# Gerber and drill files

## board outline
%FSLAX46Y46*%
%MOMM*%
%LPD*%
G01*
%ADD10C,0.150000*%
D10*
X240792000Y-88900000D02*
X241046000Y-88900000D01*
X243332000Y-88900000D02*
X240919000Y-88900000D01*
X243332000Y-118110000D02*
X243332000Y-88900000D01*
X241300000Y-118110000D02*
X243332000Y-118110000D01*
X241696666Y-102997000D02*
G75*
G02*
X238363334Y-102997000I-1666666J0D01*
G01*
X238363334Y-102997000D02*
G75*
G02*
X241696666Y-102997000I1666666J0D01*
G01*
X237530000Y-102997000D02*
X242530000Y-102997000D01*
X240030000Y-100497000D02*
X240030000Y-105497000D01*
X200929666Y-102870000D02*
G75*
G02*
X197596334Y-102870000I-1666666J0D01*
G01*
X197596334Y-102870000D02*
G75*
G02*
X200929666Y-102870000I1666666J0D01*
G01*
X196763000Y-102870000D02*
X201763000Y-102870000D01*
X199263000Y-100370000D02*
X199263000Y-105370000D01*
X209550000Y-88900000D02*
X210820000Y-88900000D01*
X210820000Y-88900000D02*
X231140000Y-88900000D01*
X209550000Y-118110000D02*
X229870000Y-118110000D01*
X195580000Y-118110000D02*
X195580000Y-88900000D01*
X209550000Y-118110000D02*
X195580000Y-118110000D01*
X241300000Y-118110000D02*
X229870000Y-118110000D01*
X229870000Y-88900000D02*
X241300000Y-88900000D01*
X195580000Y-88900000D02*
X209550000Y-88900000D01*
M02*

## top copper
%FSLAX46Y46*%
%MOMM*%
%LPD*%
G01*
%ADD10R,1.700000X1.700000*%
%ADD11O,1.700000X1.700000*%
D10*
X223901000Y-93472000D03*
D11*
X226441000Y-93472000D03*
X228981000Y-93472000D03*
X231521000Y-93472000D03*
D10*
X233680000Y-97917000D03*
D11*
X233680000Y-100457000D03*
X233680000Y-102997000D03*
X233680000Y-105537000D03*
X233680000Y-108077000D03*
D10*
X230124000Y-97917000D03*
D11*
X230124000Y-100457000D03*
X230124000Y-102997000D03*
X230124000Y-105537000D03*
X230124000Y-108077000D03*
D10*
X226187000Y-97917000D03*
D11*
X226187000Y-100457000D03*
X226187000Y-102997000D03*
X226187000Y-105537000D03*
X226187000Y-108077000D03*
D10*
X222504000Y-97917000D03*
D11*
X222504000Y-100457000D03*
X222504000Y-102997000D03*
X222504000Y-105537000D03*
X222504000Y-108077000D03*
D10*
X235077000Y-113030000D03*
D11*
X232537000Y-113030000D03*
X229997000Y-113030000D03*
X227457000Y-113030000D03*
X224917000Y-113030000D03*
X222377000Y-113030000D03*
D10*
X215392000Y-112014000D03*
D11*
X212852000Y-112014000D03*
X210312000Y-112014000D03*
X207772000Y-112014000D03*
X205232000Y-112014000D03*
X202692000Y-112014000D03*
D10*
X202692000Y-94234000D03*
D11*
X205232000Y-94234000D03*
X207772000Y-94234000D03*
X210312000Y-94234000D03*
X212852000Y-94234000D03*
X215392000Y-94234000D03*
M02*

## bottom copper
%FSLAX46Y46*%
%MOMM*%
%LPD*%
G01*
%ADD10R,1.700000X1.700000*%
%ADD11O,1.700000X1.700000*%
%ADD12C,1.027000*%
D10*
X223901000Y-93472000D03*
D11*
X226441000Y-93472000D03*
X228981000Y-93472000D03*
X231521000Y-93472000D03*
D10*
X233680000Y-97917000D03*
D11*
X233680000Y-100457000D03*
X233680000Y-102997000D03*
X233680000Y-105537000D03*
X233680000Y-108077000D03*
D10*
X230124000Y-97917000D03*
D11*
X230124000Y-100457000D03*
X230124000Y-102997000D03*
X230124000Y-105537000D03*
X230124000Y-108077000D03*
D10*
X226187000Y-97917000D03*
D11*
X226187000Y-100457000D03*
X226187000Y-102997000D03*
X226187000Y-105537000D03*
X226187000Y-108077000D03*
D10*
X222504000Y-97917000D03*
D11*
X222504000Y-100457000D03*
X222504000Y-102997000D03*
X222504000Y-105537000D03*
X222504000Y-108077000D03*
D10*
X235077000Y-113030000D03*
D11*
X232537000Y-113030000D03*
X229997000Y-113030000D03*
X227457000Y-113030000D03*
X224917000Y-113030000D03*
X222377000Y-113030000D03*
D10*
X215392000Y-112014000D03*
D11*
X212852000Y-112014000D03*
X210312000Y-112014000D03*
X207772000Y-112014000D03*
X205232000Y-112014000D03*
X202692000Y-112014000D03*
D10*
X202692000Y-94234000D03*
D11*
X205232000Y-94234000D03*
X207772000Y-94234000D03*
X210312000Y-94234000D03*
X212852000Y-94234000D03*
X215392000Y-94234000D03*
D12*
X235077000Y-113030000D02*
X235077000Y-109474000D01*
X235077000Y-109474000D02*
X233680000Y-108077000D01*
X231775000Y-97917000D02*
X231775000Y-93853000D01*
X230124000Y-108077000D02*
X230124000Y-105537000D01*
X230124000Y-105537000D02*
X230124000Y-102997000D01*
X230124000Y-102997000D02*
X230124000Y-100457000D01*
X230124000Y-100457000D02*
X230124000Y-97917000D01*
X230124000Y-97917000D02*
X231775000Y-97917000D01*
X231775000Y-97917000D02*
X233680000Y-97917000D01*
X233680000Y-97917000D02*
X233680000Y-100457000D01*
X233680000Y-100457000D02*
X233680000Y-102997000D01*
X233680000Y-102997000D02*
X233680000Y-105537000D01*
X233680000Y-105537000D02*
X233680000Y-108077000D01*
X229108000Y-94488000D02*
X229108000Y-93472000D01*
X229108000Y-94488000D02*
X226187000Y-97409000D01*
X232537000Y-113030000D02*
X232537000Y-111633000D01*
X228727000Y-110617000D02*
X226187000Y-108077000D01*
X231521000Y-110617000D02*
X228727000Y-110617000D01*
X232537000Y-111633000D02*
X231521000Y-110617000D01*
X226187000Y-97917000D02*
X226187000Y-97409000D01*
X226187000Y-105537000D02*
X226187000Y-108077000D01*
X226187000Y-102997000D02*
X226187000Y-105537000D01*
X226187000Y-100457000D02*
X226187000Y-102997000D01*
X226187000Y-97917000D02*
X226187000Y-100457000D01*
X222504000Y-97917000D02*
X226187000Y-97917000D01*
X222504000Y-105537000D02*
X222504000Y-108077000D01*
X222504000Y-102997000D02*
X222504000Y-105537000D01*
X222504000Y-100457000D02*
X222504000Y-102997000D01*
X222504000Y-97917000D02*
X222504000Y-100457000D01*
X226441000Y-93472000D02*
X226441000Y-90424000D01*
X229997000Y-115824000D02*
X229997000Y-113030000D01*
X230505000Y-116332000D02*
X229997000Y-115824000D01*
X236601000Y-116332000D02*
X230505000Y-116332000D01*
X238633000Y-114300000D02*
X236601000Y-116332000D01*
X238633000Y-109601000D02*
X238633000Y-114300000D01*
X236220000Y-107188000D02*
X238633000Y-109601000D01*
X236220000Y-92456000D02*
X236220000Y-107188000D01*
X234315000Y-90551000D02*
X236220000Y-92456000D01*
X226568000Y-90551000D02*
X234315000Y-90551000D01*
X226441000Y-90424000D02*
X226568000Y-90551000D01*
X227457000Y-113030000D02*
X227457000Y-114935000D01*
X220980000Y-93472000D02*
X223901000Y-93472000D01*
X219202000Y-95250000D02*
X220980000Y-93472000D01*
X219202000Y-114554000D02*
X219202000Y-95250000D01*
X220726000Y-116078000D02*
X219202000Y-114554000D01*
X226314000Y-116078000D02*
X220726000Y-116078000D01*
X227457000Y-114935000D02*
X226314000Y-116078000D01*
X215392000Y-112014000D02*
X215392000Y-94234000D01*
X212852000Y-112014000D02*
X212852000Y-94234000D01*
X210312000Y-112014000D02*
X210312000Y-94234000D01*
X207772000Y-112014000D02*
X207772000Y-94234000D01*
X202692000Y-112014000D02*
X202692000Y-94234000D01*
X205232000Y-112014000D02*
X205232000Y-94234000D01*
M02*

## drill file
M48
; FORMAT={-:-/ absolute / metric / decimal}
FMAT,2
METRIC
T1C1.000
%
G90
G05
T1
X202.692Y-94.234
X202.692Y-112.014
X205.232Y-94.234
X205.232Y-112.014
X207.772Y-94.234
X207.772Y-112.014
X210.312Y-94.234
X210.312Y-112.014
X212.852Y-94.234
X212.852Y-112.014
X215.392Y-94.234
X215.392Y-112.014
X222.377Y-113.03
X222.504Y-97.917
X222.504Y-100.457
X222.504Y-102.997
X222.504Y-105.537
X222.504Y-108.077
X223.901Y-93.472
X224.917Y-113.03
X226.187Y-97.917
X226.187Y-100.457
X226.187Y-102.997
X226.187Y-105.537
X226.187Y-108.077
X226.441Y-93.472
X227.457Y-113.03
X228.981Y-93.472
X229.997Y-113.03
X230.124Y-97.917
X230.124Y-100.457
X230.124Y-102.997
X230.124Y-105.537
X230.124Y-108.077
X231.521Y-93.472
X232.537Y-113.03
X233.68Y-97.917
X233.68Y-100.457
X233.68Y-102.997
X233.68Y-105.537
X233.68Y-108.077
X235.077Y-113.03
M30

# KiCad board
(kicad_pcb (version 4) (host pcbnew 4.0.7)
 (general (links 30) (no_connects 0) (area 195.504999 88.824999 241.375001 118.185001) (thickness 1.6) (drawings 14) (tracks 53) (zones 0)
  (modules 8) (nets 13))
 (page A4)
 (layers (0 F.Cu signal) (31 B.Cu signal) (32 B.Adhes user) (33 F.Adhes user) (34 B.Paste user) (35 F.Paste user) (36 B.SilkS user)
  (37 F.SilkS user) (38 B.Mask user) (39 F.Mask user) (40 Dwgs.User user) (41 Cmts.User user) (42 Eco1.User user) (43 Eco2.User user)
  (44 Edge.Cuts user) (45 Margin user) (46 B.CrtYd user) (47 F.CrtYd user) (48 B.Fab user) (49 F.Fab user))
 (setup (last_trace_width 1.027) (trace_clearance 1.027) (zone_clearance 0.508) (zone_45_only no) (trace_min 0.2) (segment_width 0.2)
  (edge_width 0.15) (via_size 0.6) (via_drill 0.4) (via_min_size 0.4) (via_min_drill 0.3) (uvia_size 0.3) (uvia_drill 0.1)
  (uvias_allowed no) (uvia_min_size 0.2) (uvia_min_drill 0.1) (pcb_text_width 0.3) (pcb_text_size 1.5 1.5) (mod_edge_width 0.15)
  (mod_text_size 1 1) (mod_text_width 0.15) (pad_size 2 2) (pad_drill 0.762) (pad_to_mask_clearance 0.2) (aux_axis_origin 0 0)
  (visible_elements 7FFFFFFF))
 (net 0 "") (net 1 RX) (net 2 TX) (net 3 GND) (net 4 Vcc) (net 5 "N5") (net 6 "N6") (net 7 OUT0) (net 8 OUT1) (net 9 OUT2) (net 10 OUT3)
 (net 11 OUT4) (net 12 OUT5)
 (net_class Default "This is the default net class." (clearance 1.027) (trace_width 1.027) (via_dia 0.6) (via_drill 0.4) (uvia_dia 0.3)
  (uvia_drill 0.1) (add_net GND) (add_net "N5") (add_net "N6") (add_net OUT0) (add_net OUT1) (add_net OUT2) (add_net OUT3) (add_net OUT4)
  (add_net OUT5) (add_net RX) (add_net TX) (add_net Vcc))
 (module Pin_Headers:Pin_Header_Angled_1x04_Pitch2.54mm (layer F.Cu) (at 223.901 93.472 90)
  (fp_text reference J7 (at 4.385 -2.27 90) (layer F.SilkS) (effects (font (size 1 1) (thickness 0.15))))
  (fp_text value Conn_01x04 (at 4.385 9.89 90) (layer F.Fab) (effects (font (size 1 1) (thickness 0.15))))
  (pad 1 thru_hole rect (at 0 0 90) (size 1.7 1.7) (drill 1) (layers *.Cu *.Mask) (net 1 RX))
  (pad 2 thru_hole oval (at 0 2.54 90) (size 1.7 1.7) (drill 1) (layers *.Cu *.Mask) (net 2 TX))
  (pad 3 thru_hole oval (at 0 5.08 90) (size 1.7 1.7) (drill 1) (layers *.Cu *.Mask) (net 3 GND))
  (pad 4 thru_hole oval (at 0 7.62 90) (size 1.7 1.7) (drill 1) (layers *.Cu *.Mask) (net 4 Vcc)))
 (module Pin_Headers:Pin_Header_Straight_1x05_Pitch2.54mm (layer F.Cu) (at 233.68 97.917)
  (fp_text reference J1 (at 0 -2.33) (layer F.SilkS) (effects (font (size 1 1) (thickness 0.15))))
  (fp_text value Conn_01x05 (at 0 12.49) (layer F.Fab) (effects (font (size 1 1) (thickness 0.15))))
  (pad 1 thru_hole rect (at 0 0) (size 1.7 1.7) (drill 1) (layers *.Cu *.Mask) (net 4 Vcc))
  (pad 2 thru_hole oval (at 0 2.54) (size 1.7 1.7) (drill 1) (layers *.Cu *.Mask) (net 4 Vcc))
  (pad 3 thru_hole oval (at 0 5.08) (size 1.7 1.7) (drill 1) (layers *.Cu *.Mask) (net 4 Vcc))
  (pad 4 thru_hole oval (at 0 7.62) (size 1.7 1.7) (drill 1) (layers *.Cu *.Mask) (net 4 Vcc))
  (pad 5 thru_hole oval (at 0 10.16) (size 1.7 1.7) (drill 1) (layers *.Cu *.Mask) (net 4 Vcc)))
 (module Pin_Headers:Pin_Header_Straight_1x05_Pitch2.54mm (layer F.Cu) (at 230.124 97.917)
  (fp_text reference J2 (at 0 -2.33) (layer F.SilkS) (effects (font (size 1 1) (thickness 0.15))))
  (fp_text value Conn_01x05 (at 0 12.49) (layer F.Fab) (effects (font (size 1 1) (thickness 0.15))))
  (pad 1 thru_hole rect (at 0 0) (size 1.7 1.7) (drill 1) (layers *.Cu *.Mask) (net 4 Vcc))
  (pad 2 thru_hole oval (at 0 2.54) (size 1.7 1.7) (drill 1) (layers *.Cu *.Mask) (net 4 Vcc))
  (pad 3 thru_hole oval (at 0 5.08) (size 1.7 1.7) (drill 1) (layers *.Cu *.Mask) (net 4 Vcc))
  (pad 4 thru_hole oval (at 0 7.62) (size 1.7 1.7) (drill 1) (layers *.Cu *.Mask) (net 4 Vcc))
  (pad 5 thru_hole oval (at 0 10.16) (size 1.7 1.7) (drill 1) (layers *.Cu *.Mask) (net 4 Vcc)))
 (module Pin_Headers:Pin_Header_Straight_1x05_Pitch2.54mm (layer F.Cu) (at 226.187 97.917)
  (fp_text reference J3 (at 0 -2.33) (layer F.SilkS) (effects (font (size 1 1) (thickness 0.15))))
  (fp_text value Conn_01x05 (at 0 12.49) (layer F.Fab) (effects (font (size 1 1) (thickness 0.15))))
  (pad 1 thru_hole rect (at 0 0) (size 1.7 1.7) (drill 1) (layers *.Cu *.Mask) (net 3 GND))
  (pad 2 thru_hole oval (at 0 2.54) (size 1.7 1.7) (drill 1) (layers *.Cu *.Mask) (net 3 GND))
  (pad 3 thru_hole oval (at 0 5.08) (size 1.7 1.7) (drill 1) (layers *.Cu *.Mask) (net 3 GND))
  (pad 4 thru_hole oval (at 0 7.62) (size 1.7 1.7) (drill 1) (layers *.Cu *.Mask) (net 3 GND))
  (pad 5 thru_hole oval (at 0 10.16) (size 1.7 1.7) (drill 1) (layers *.Cu *.Mask) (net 3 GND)))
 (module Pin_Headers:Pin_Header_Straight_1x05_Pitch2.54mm (layer F.Cu) (at 222.504 97.917)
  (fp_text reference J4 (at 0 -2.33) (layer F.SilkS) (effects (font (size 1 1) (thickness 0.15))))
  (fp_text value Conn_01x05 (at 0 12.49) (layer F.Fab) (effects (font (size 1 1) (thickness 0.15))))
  (pad 1 thru_hole rect (at 0 0) (size 1.7 1.7) (drill 1) (layers *.Cu *.Mask) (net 3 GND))
  (pad 2 thru_hole oval (at 0 2.54) (size 1.7 1.7) (drill 1) (layers *.Cu *.Mask) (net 3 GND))
  (pad 3 thru_hole oval (at 0 5.08) (size 1.7 1.7) (drill 1) (layers *.Cu *.Mask) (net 3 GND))
  (pad 4 thru_hole oval (at 0 7.62) (size 1.7 1.7) (drill 1) (layers *.Cu *.Mask) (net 3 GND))
  (pad 5 thru_hole oval (at 0 10.16) (size 1.7 1.7) (drill 1) (layers *.Cu *.Mask) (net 3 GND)))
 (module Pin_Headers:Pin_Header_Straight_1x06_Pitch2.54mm (layer F.Cu) (at 235.077 113.03 270)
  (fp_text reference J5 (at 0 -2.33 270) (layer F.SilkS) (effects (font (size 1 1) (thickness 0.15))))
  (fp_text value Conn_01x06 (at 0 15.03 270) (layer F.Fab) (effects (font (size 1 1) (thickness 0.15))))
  (pad 1 thru_hole rect (at 0 0 270) (size 1.7 1.7) (drill 1) (layers *.Cu *.Mask) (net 4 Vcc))
  (pad 2 thru_hole oval (at 0 2.54 270) (size 1.7 1.7) (drill 1) (layers *.Cu *.Mask) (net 3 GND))
  (pad 3 thru_hole oval (at 0 5.08 270) (size 1.7 1.7) (drill 1) (layers *.Cu *.Mask) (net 2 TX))
  (pad 4 thru_hole oval (at 0 7.62 270) (size 1.7 1.7) (drill 1) (layers *.Cu *.Mask) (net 1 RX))
  (pad 5 thru_hole oval (at 0 10.16 270) (size 1.7 1.7) (drill 1) (layers *.Cu *.Mask) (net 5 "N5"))
  (pad 6 thru_hole oval (at 0 12.7 270) (size 1.7 1.7) (drill 1) (layers *.Cu *.Mask) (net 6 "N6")))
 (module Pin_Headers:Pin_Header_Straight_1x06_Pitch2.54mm (layer F.Cu) (at 215.392 112.014 270)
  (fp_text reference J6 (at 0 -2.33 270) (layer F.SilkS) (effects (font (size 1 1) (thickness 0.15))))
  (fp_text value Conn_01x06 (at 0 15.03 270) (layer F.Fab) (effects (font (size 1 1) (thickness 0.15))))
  (pad 1 thru_hole rect (at 0 0 270) (size 1.7 1.7) (drill 1) (layers *.Cu *.Mask) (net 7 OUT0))
  (pad 2 thru_hole oval (at 0 2.54 270) (size 1.7 1.7) (drill 1) (layers *.Cu *.Mask) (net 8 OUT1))
  (pad 3 thru_hole oval (at 0 5.08 270) (size 1.7 1.7) (drill 1) (layers *.Cu *.Mask) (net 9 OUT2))
  (pad 4 thru_hole oval (at 0 7.62 270) (size 1.7 1.7) (drill 1) (layers *.Cu *.Mask) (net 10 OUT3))
  (pad 5 thru_hole oval (at 0 10.16 270) (size 1.7 1.7) (drill 1) (layers *.Cu *.Mask) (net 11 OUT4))
  (pad 6 thru_hole oval (at 0 12.7 270) (size 1.7 1.7) (drill 1) (layers *.Cu *.Mask) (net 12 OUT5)))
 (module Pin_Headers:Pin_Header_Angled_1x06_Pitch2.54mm (layer F.Cu) (at 202.692 94.234 90)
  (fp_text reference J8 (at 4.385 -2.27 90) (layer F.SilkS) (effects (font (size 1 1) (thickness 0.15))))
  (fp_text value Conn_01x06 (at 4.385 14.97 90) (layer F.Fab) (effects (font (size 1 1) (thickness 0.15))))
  (pad 1 thru_hole rect (at 0 0 90) (size 1.7 1.7) (drill 1) (layers *.Cu *.Mask) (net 12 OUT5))
  (pad 2 thru_hole oval (at 0 2.54 90) (size 1.7 1.7) (drill 1) (layers *.Cu *.Mask) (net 11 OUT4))
  (pad 3 thru_hole oval (at 0 5.08 90) (size 1.7 1.7) (drill 1) (layers *.Cu *.Mask) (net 10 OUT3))
  (pad 4 thru_hole oval (at 0 7.62 90) (size 1.7 1.7) (drill 1) (layers *.Cu *.Mask) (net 9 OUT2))
  (pad 5 thru_hole oval (at 0 10.16 90) (size 1.7 1.7) (drill 1) (layers *.Cu *.Mask) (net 8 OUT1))
  (pad 6 thru_hole oval (at 0 12.7 90) (size 1.7 1.7) (drill 1) (layers *.Cu *.Mask) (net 7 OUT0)))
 (gr_line (start 240.792 88.9) (end 241.046 88.9) (angle 90) (layer Edge.Cuts) (width 0.15))
 (gr_line (start 243.332 88.9) (end 240.919 88.9) (angle 90) (layer Edge.Cuts) (width 0.15))
 (gr_line (start 243.332 118.11) (end 243.332 88.9) (angle 90) (layer Edge.Cuts) (width 0.15))
 (gr_line (start 241.3 118.11) (end 243.332 118.11) (angle 90) (layer Edge.Cuts) (width 0.15))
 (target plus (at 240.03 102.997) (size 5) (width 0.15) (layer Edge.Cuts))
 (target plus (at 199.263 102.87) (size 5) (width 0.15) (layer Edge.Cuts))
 (gr_line (start 209.55 88.9) (end 210.82 88.9) (angle 90) (layer Edge.Cuts) (width 0.15))
 (gr_line (start 210.82 88.9) (end 231.14 88.9) (angle 90) (layer Edge.Cuts) (width 0.15))
 (gr_line (start 209.55 118.11) (end 229.87 118.11) (angle 90) (layer Edge.Cuts) (width 0.15))
 (gr_line (start 195.58 118.11) (end 195.58 88.9) (angle 90) (layer Edge.Cuts) (width 0.15))
 (gr_line (start 209.55 118.11) (end 195.58 118.11) (angle 90) (layer Edge.Cuts) (width 0.15))
 (gr_line (start 241.3 118.11) (end 229.87 118.11) (angle 90) (layer Edge.Cuts) (width 0.15))
 (gr_line (start 229.87 88.9) (end 241.3 88.9) (angle 90) (layer Edge.Cuts) (width 0.15))
 (gr_line (start 195.58 88.9) (end 209.55 88.9) (angle 90) (layer Edge.Cuts) (width 0.15))
 (segment (start 235.077 113.03) (end 235.077 109.474) (width 1.027) (layer B.Cu) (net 4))
 (segment (start 235.077 109.474) (end 233.68 108.077) (width 1.027) (layer B.Cu) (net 4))
 (segment (start 231.775 97.917) (end 231.775 93.853) (width 1.027) (layer B.Cu) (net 4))
 (segment (start 230.124 108.077) (end 230.124 105.537) (width 1.027) (layer B.Cu) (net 4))
 (segment (start 230.124 105.537) (end 230.124 102.997) (width 1.027) (layer B.Cu) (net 4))
 (segment (start 230.124 102.997) (end 230.124 100.457) (width 1.027) (layer B.Cu) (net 4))
 (segment (start 230.124 100.457) (end 230.124 97.917) (width 1.027) (layer B.Cu) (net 4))
 (segment (start 230.124 97.917) (end 231.775 97.917) (width 1.027) (layer B.Cu) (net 4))
 (segment (start 231.775 97.917) (end 233.68 97.917) (width 1.027) (layer B.Cu) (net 4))
 (segment (start 233.68 97.917) (end 233.68 100.457) (width 1.027) (layer B.Cu) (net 4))
 (segment (start 233.68 100.457) (end 233.68 102.997) (width 1.027) (layer B.Cu) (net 4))
 (segment (start 233.68 102.997) (end 233.68 105.537) (width 1.027) (layer B.Cu) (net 4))
 (segment (start 233.68 105.537) (end 233.68 108.077) (width 1.027) (layer B.Cu) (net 4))
 (segment (start 229.108 94.488) (end 229.108 93.472) (width 1.027) (layer B.Cu) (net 3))
 (segment (start 229.108 94.488) (end 226.187 97.409) (width 1.027) (layer B.Cu) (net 3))
 (segment (start 232.537 113.03) (end 232.537 111.633) (width 1.027) (layer B.Cu) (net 3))
 (segment (start 228.727 110.617) (end 226.187 108.077) (width 1.027) (layer B.Cu) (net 3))
 (segment (start 231.521 110.617) (end 228.727 110.617) (width 1.027) (layer B.Cu) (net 3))
 (segment (start 232.537 111.633) (end 231.521 110.617) (width 1.027) (layer B.Cu) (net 3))
 (segment (start 226.187 97.917) (end 226.187 97.409) (width 1.027) (layer B.Cu) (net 3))
 (segment (start 226.187 105.537) (end 226.187 108.077) (width 1.027) (layer B.Cu) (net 3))
 (segment (start 226.187 102.997) (end 226.187 105.537) (width 1.027) (layer B.Cu) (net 3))
 (segment (start 226.187 100.457) (end 226.187 102.997) (width 1.027) (layer B.Cu) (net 3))
 (segment (start 226.187 97.917) (end 226.187 100.457) (width 1.027) (layer B.Cu) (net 3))
 (segment (start 222.504 97.917) (end 226.187 97.917) (width 1.027) (layer B.Cu) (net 3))
 (segment (start 222.504 105.537) (end 222.504 108.077) (width 1.027) (layer B.Cu) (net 3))
 (segment (start 222.504 102.997) (end 222.504 105.537) (width 1.027) (layer B.Cu) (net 3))
 (segment (start 222.504 100.457) (end 222.504 102.997) (width 1.027) (layer B.Cu) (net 3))
 (segment (start 222.504 97.917) (end 222.504 100.457) (width 1.027) (layer B.Cu) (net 3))
 (segment (start 226.441 93.472) (end 226.441 90.424) (width 1.027) (layer B.Cu) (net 2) (status 400000))
 (segment (start 229.997 115.824) (end 229.997 113.03) (width 1.027) (layer B.Cu) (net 2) (status 800000))
 (segment (start 230.505 116.332) (end 229.997 115.824) (width 1.027) (layer B.Cu) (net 2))
 (segment (start 236.601 116.332) (end 230.505 116.332) (width 1.027) (layer B.Cu) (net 2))
 (segment (start 238.633 114.3) (end 236.601 116.332) (width 1.027) (layer B.Cu) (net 2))
 (segment (start 238.633 109.601) (end 238.633 114.3) (width 1.027) (layer B.Cu) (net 2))
 (segment (start 236.22 107.188) (end 238.633 109.601) (width 1.027) (layer B.Cu) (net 2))
 (segment (start 236.22 92.456) (end 236.22 107.188) (width 1.027) (layer B.Cu) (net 2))
 (segment (start 234.315 90.551) (end 236.22 92.456) (width 1.027) (layer B.Cu) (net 2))
 (segment (start 226.568 90.551) (end 234.315 90.551) (width 1.027) (layer B.Cu) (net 2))
 (segment (start 226.441 90.424) (end 226.568 90.551) (width 1.027) (layer B.Cu) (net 2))
 (segment (start 227.457 113.03) (end 227.457 114.935) (width 1.027) (layer B.Cu) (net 1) (status 400000))
 (segment (start 220.98 93.472) (end 223.901 93.472) (width 1.027) (layer B.Cu) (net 1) (status 800000))
 (segment (start 219.202 95.25) (end 220.98 93.472) (width 1.027) (layer B.Cu) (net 1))
 (segment (start 219.202 114.554) (end 219.202 95.25) (width 1.027) (layer B.Cu) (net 1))
 (segment (start 220.726 116.078) (end 219.202 114.554) (width 1.027) (layer B.Cu) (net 1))
 (segment (start 226.314 116.078) (end 220.726 116.078) (width 1.027) (layer B.Cu) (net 1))
 (segment (start 227.457 114.935) (end 226.314 116.078) (width 1.027) (layer B.Cu) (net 1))
 (segment (start 215.392 112.014) (end 215.392 94.234) (width 1.027) (layer B.Cu) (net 7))
 (segment (start 212.852 112.014) (end 212.852 94.234) (width 1.027) (layer B.Cu) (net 8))
 (segment (start 210.312 112.014) (end 210.312 94.234) (width 1.027) (layer B.Cu) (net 9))
 (segment (start 207.772 112.014) (end 207.772 94.234) (width 1.027) (layer B.Cu) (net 10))
 (segment (start 202.692 112.014) (end 202.692 94.234) (width 1.027) (layer B.Cu) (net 12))
 (segment (start 205.232 112.014) (end 205.232 94.234) (width 1.027) (layer B.Cu) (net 11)))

